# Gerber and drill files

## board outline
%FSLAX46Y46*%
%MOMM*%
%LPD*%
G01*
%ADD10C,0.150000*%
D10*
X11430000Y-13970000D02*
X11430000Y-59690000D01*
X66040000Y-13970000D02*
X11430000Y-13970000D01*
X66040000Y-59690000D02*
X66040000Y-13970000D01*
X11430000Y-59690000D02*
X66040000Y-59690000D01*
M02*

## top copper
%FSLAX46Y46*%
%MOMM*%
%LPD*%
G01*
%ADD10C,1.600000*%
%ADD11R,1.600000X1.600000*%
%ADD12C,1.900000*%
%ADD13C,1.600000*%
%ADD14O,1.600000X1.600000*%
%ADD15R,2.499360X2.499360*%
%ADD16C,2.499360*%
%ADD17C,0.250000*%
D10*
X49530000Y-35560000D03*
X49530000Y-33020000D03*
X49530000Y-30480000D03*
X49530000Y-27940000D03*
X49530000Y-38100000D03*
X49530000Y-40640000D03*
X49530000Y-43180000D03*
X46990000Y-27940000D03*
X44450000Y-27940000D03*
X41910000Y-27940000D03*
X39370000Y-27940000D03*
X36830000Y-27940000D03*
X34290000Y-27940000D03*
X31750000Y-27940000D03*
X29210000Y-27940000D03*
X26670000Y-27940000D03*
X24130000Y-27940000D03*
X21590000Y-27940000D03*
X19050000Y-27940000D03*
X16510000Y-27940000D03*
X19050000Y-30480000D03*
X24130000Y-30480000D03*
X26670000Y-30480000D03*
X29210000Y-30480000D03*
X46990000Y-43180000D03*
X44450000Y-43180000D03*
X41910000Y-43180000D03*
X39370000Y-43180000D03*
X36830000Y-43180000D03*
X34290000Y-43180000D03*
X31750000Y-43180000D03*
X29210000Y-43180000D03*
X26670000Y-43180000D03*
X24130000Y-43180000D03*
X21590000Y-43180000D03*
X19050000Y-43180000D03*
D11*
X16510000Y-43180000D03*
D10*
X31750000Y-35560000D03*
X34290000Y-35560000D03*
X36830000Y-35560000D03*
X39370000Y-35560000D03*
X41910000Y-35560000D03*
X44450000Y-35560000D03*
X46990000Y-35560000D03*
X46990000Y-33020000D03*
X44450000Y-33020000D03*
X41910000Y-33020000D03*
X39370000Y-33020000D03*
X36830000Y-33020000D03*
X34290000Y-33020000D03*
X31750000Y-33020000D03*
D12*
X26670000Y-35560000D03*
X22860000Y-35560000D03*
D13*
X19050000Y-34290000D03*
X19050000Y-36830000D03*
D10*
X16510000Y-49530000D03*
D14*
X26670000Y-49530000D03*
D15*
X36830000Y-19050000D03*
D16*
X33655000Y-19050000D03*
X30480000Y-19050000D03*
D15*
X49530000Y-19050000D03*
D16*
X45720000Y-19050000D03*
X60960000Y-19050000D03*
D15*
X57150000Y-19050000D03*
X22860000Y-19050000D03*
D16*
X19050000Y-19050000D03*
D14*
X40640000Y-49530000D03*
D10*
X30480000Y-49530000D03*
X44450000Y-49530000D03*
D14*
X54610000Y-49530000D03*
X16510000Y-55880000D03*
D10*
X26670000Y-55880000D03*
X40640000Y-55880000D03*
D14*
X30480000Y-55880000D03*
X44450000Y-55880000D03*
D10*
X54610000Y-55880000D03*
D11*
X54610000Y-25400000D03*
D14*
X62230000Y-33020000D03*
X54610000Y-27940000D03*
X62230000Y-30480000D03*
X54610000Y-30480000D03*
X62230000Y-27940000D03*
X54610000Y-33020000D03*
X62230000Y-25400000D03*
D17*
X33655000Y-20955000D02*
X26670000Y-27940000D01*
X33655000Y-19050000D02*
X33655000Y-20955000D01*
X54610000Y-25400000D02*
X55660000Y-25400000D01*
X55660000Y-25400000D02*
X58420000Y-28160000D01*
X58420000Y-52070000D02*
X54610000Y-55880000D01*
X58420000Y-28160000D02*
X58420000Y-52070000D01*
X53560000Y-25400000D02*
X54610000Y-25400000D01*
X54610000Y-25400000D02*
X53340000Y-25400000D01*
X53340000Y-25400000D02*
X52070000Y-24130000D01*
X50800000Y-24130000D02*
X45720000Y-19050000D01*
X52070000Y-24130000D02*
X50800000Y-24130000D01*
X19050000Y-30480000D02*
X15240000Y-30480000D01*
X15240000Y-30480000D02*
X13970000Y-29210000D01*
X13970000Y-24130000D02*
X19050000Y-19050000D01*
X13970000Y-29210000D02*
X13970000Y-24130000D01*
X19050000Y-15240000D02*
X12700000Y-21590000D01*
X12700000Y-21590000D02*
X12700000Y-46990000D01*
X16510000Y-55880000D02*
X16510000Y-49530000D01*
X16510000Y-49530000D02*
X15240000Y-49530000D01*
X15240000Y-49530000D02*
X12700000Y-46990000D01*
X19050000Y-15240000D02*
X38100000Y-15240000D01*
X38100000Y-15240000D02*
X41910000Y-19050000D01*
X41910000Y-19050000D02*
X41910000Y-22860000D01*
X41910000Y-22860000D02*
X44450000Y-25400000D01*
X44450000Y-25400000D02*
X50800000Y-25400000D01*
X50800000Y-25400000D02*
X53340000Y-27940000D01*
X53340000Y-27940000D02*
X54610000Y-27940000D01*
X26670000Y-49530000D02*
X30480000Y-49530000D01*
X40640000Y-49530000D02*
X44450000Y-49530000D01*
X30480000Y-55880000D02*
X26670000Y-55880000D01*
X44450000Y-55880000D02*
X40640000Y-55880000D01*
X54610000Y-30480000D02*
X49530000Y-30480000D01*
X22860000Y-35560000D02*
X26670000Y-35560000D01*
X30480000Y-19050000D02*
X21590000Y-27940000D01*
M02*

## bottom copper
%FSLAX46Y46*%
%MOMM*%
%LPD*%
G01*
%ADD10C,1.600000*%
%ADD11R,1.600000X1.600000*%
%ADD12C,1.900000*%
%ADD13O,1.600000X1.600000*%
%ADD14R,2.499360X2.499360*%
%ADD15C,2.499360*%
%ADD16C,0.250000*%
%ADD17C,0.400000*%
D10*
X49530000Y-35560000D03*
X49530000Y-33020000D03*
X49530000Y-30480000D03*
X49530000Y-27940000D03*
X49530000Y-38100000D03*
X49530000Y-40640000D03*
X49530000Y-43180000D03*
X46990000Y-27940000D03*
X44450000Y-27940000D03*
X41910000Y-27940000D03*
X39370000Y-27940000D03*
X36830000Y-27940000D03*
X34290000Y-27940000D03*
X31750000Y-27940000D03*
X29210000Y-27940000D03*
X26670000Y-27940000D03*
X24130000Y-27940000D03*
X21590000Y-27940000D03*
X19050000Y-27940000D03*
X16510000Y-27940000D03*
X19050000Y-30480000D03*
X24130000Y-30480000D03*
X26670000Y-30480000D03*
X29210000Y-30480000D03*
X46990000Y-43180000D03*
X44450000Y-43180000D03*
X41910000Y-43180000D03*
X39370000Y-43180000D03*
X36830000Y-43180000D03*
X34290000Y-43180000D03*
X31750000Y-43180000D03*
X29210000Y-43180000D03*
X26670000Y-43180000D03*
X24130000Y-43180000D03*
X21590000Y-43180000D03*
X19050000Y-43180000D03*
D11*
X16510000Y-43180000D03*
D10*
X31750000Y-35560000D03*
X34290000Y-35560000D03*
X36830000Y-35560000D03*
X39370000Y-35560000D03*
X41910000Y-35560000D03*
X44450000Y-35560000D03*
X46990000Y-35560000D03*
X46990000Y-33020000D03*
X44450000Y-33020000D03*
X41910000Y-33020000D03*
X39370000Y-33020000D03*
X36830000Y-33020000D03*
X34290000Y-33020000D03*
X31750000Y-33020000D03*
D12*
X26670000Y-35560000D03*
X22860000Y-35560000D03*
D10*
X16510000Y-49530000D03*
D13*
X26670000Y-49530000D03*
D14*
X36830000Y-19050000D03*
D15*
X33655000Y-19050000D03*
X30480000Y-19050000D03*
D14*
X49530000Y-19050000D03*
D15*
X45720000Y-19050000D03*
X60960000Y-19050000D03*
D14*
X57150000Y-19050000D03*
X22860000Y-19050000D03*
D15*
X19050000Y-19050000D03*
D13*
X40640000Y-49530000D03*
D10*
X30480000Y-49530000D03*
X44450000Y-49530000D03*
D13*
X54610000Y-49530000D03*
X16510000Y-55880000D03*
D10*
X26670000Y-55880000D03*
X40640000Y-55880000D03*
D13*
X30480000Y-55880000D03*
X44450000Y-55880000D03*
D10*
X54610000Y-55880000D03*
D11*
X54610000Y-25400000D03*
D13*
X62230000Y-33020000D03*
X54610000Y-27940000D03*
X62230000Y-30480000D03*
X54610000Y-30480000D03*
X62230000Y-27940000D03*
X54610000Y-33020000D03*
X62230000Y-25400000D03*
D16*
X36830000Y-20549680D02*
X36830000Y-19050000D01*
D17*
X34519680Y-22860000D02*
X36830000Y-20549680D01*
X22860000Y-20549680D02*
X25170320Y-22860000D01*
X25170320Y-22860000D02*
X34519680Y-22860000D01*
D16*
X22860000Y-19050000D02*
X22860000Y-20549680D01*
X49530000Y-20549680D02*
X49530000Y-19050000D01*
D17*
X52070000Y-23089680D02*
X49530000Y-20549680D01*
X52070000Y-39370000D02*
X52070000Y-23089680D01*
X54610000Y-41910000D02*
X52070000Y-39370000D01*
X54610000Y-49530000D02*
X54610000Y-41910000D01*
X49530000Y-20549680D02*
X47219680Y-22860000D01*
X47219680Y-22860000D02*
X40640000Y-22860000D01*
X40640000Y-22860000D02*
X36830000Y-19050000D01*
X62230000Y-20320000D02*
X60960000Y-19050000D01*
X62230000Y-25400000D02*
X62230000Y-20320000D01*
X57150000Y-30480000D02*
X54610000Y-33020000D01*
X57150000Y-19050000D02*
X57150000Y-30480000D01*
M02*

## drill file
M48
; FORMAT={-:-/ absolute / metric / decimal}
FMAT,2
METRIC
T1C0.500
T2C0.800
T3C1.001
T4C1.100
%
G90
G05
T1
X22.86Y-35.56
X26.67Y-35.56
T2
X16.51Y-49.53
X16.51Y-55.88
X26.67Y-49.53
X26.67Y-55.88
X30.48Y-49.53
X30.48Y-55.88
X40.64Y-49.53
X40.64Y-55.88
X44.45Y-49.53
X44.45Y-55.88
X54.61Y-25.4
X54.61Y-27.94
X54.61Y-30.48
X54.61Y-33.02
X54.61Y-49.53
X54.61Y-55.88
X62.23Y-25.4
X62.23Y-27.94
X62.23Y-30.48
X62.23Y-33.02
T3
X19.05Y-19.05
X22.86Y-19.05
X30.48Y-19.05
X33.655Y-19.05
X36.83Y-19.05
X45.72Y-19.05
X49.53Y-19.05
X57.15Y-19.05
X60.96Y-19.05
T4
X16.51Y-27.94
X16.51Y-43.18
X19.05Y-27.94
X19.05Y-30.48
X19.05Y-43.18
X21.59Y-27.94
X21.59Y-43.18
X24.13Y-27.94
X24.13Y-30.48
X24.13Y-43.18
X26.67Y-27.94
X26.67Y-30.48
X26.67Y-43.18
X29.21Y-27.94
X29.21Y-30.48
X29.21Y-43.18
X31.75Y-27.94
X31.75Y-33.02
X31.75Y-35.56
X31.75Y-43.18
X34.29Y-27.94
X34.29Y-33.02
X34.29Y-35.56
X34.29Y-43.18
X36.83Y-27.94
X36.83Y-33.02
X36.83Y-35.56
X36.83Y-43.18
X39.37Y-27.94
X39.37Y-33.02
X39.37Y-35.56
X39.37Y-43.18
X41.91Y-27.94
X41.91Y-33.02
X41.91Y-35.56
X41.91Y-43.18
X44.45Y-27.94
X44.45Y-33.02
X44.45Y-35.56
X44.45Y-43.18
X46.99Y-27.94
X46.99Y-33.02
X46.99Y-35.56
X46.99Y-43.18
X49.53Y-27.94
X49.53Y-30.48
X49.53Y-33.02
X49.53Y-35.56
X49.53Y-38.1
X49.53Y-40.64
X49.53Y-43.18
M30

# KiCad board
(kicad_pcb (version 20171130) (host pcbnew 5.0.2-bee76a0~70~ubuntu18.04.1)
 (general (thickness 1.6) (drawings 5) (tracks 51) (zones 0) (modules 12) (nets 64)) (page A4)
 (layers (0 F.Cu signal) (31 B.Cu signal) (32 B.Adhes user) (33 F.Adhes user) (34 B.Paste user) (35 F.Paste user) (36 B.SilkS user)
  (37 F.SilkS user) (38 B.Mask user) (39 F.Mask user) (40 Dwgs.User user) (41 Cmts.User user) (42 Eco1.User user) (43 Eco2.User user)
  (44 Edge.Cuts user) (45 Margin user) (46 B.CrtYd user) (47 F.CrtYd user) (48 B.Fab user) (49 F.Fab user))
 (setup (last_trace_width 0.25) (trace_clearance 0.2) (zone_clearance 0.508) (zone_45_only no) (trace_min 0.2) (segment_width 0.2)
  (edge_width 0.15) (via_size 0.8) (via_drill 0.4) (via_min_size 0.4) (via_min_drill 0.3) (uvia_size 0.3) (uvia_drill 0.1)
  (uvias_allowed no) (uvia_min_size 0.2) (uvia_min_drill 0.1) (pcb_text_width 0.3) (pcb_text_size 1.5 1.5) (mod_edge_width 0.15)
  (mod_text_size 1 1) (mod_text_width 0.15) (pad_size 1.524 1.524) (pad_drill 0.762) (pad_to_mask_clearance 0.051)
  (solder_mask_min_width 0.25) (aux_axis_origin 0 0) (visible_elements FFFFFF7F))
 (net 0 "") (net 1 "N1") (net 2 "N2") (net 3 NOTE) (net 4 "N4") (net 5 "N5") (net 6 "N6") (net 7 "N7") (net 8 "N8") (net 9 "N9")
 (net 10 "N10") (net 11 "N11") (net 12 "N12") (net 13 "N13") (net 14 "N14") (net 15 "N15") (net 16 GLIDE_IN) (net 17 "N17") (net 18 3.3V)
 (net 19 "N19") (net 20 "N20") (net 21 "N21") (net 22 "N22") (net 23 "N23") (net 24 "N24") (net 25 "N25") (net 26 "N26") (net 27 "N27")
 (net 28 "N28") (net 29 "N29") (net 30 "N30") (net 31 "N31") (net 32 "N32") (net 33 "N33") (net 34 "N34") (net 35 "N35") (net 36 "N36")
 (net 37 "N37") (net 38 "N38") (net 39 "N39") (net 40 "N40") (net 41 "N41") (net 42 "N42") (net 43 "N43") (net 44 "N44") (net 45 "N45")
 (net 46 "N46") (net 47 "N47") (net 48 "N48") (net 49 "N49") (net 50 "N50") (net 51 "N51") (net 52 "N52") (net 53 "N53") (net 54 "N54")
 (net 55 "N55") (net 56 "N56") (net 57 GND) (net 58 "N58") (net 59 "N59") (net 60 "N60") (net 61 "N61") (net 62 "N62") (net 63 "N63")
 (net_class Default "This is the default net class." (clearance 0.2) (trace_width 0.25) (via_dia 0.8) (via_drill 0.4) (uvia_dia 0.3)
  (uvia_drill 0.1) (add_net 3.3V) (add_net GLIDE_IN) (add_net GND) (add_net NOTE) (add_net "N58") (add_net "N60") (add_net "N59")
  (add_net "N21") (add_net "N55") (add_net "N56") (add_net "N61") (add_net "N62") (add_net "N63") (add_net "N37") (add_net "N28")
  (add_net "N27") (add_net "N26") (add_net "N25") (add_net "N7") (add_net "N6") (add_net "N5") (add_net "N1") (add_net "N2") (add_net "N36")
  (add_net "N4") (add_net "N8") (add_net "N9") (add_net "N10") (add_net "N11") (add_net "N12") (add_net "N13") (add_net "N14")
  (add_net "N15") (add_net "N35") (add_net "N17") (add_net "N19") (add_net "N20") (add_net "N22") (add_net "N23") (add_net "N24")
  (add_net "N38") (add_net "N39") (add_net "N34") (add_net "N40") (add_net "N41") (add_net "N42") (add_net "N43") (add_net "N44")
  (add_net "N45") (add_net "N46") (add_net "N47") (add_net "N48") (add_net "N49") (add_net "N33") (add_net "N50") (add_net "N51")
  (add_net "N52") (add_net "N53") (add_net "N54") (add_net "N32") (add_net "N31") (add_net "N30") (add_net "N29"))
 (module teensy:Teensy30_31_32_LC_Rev (layer F.Cu) (at 33.02 35.56)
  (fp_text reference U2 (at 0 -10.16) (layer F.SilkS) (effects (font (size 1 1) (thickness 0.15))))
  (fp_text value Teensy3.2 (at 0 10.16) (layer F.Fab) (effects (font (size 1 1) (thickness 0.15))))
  (pad 17 thru_hole circle (at 16.51 0) (size 1.6 1.6) (drill 1.1) (layers *.Cu *.Mask F.SilkS) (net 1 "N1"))
  (pad 18 thru_hole circle (at 16.51 -2.54) (size 1.6 1.6) (drill 1.1) (layers *.Cu *.Mask F.SilkS) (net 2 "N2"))
  (pad 19 thru_hole circle (at 16.51 -5.08) (size 1.6 1.6) (drill 1.1) (layers *.Cu *.Mask F.SilkS) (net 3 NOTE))
  (pad 20 thru_hole circle (at 16.51 -7.62) (size 1.6 1.6) (drill 1.1) (layers *.Cu *.Mask F.SilkS) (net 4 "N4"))
  (pad 16 thru_hole circle (at 16.51 2.54) (size 1.6 1.6) (drill 1.1) (layers *.Cu *.Mask F.SilkS) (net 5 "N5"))
  (pad 15 thru_hole circle (at 16.51 5.08) (size 1.6 1.6) (drill 1.1) (layers *.Cu *.Mask F.SilkS) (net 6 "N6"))
  (pad 14 thru_hole circle (at 16.51 7.62) (size 1.6 1.6) (drill 1.1) (layers *.Cu *.Mask F.SilkS) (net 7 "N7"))
  (pad 21 thru_hole circle (at 13.97 -7.62) (size 1.6 1.6) (drill 1.1) (layers *.Cu *.Mask F.SilkS) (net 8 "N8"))
  (pad 22 thru_hole circle (at 11.43 -7.62) (size 1.6 1.6) (drill 1.1) (layers *.Cu *.Mask F.SilkS) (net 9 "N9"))
  (pad 23 thru_hole circle (at 8.89 -7.62) (size 1.6 1.6) (drill 1.1) (layers *.Cu *.Mask F.SilkS) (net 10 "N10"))
  (pad 24 thru_hole circle (at 6.35 -7.62) (size 1.6 1.6) (drill 1.1) (layers *.Cu *.Mask F.SilkS) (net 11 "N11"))
  (pad 25 thru_hole circle (at 3.81 -7.62) (size 1.6 1.6) (drill 1.1) (layers *.Cu *.Mask F.SilkS) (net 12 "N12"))
  (pad 26 thru_hole circle (at 1.27 -7.62) (size 1.6 1.6) (drill 1.1) (layers *.Cu *.Mask F.SilkS) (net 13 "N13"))
  (pad 27 thru_hole circle (at -1.27 -7.62) (size 1.6 1.6) (drill 1.1) (layers *.Cu *.Mask F.SilkS) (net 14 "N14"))
  (pad 28 thru_hole circle (at -3.81 -7.62) (size 1.6 1.6) (drill 1.1) (layers *.Cu *.Mask F.SilkS) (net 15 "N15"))
  (pad 29 thru_hole circle (at -6.35 -7.62) (size 1.6 1.6) (drill 1.1) (layers *.Cu *.Mask F.SilkS) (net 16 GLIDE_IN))
  (pad 30 thru_hole circle (at -8.89 -7.62) (size 1.6 1.6) (drill 1.1) (layers *.Cu *.Mask F.SilkS) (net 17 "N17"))
  (pad 31 thru_hole circle (at -11.43 -7.62) (size 1.6 1.6) (drill 1.1) (layers *.Cu *.Mask F.SilkS) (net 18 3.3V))
  (pad 32 thru_hole circle (at -13.97 -7.62) (size 1.6 1.6) (drill 1.1) (layers *.Cu *.Mask F.SilkS) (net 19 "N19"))
  (pad 33 thru_hole circle (at -16.51 -7.62) (size 1.6 1.6) (drill 1.1) (layers *.Cu *.Mask F.SilkS) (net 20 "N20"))
  (pad 34 thru_hole circle (at -13.97 -5.08) (size 1.6 1.6) (drill 1.1) (layers *.Cu *.Mask F.SilkS) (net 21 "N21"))
  (pad 35 thru_hole circle (at -8.89 -5.08) (size 1.6 1.6) (drill 1.1) (layers *.Cu *.Mask F.SilkS) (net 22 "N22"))
  (pad 36 thru_hole circle (at -6.35 -5.08) (size 1.6 1.6) (drill 1.1) (layers *.Cu *.Mask F.SilkS) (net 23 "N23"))
  (pad 37 thru_hole circle (at -3.81 -5.08) (size 1.6 1.6) (drill 1.1) (layers *.Cu *.Mask F.SilkS) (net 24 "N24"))
  (pad 13 thru_hole circle (at 13.97 7.62) (size 1.6 1.6) (drill 1.1) (layers *.Cu *.Mask F.SilkS) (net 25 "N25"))
  (pad 12 thru_hole circle (at 11.43 7.62) (size 1.6 1.6) (drill 1.1) (layers *.Cu *.Mask F.SilkS) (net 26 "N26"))
  (pad 11 thru_hole circle (at 8.89 7.62) (size 1.6 1.6) (drill 1.1) (layers *.Cu *.Mask F.SilkS) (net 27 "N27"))
  (pad 10 thru_hole circle (at 6.35 7.62) (size 1.6 1.6) (drill 1.1) (layers *.Cu *.Mask F.SilkS) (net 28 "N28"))
  (pad 9 thru_hole circle (at 3.81 7.62) (size 1.6 1.6) (drill 1.1) (layers *.Cu *.Mask F.SilkS) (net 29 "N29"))
  (pad 8 thru_hole circle (at 1.27 7.62) (size 1.6 1.6) (drill 1.1) (layers *.Cu *.Mask F.SilkS) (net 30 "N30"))
  (pad 7 thru_hole circle (at -1.27 7.62) (size 1.6 1.6) (drill 1.1) (layers *.Cu *.Mask F.SilkS) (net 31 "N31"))
  (pad 6 thru_hole circle (at -3.81 7.62) (size 1.6 1.6) (drill 1.1) (layers *.Cu *.Mask F.SilkS) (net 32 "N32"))
  (pad 5 thru_hole circle (at -6.35 7.62) (size 1.6 1.6) (drill 1.1) (layers *.Cu *.Mask F.SilkS) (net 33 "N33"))
  (pad 4 thru_hole circle (at -8.89 7.62) (size 1.6 1.6) (drill 1.1) (layers *.Cu *.Mask F.SilkS) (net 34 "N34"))
  (pad 3 thru_hole circle (at -11.43 7.62) (size 1.6 1.6) (drill 1.1) (layers *.Cu *.Mask F.SilkS) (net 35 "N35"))
  (pad 2 thru_hole circle (at -13.97 7.62) (size 1.6 1.6) (drill 1.1) (layers *.Cu *.Mask F.SilkS) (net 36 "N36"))
  (pad 1 thru_hole rect (at -16.51 7.62) (size 1.6 1.6) (drill 1.1) (layers *.Cu *.Mask F.SilkS) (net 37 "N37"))
  (pad 38 thru_hole circle (at -1.27 0) (size 1.6 1.6) (drill 1.1) (layers *.Cu *.Mask) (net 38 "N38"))
  (pad 39 thru_hole circle (at 1.27 0) (size 1.6 1.6) (drill 1.1) (layers *.Cu *.Mask) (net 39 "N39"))
  (pad 40 thru_hole circle (at 3.81 0) (size 1.6 1.6) (drill 1.1) (layers *.Cu *.Mask) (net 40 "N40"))
  (pad 41 thru_hole circle (at 6.35 0) (size 1.6 1.6) (drill 1.1) (layers *.Cu *.Mask) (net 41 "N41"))
  (pad 42 thru_hole circle (at 8.89 0) (size 1.6 1.6) (drill 1.1) (layers *.Cu *.Mask) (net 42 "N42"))
  (pad 43 thru_hole circle (at 11.43 0) (size 1.6 1.6) (drill 1.1) (layers *.Cu *.Mask) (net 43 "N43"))
  (pad 44 thru_hole circle (at 13.97 0) (size 1.6 1.6) (drill 1.1) (layers *.Cu *.Mask) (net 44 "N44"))
  (pad 45 thru_hole circle (at 13.97 -2.54) (size 1.6 1.6) (drill 1.1) (layers *.Cu *.Mask) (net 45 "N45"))
  (pad 46 thru_hole circle (at 11.43 -2.54) (size 1.6 1.6) (drill 1.1) (layers *.Cu *.Mask) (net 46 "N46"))
  (pad 47 thru_hole circle (at 8.89 -2.54) (size 1.6 1.6) (drill 1.1) (layers *.Cu *.Mask) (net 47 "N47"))
  (pad 48 thru_hole circle (at 6.35 -2.54) (size 1.6 1.6) (drill 1.1) (layers *.Cu *.Mask) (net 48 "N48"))
  (pad 49 thru_hole circle (at 3.81 -2.54) (size 1.6 1.6) (drill 1.1) (layers *.Cu *.Mask) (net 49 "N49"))
  (pad 50 thru_hole circle (at 1.27 -2.54) (size 1.6 1.6) (drill 1.1) (layers *.Cu *.Mask) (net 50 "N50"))
  (pad 51 thru_hole circle (at -1.27 -2.54) (size 1.6 1.6) (drill 1.1) (layers *.Cu *.Mask) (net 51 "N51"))
  (pad 52 thru_hole circle (at -6.35 0) (size 1.9 1.9) (drill 0.5) (layers *.Cu *.Mask F.SilkS) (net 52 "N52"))
  (pad 52 thru_hole circle (at -10.16 0) (size 1.9 1.9) (drill 0.5) (layers *.Cu *.Mask F.SilkS) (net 52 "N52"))
  (pad 53 smd circle (at -13.97 -1.27) (size 1.6 1.6) (layers F.Cu F.Paste F.Mask) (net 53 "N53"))
  (pad 54 smd circle (at -13.97 1.27) (size 1.6 1.6) (layers F.Cu F.Paste F.Mask) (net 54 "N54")))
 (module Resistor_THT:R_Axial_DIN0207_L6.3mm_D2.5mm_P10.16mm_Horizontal (layer F.Cu) (at 16.51 49.53)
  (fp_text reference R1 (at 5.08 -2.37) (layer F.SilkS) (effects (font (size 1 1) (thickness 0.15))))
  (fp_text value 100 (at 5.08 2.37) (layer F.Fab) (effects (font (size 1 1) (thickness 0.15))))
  (pad 1 thru_hole circle (at 0 0) (size 1.6 1.6) (drill 0.8) (layers *.Cu *.Mask) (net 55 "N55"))
  (pad 2 thru_hole oval (at 10.16 0) (size 1.6 1.6) (drill 0.8) (layers *.Cu *.Mask) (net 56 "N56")))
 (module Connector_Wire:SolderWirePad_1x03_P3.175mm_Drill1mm (layer F.Cu) (at 36.83 19.05 180)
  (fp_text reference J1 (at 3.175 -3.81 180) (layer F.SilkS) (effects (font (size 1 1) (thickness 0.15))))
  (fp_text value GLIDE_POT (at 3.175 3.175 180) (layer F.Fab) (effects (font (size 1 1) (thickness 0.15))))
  (pad 1 thru_hole rect (at 0 0 180) (size 2.49936 2.49936) (drill 1.00076) (layers *.Cu *.Mask) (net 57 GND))
  (pad 2 thru_hole circle (at 3.175 0 180) (size 2.49936 2.49936) (drill 1.00076) (layers *.Cu *.Mask) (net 16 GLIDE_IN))
  (pad 3 thru_hole circle (at 6.35 0 180) (size 2.49936 2.49936) (drill 1.00076) (layers *.Cu *.Mask) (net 18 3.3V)))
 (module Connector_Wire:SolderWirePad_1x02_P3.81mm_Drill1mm (layer F.Cu) (at 49.53 19.05 180)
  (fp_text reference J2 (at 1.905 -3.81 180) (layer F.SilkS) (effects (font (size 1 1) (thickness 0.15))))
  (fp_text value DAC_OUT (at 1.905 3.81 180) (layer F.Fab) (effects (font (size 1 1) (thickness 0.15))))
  (pad 1 thru_hole rect (at 0 0 180) (size 2.49936 2.49936) (drill 1.00076) (layers *.Cu *.Mask) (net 57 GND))
  (pad 2 thru_hole circle (at 3.81 0 180) (size 2.49936 2.49936) (drill 1.00076) (layers *.Cu *.Mask) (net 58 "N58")))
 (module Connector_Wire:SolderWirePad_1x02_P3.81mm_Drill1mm (layer F.Cu) (at 57.15 19.05)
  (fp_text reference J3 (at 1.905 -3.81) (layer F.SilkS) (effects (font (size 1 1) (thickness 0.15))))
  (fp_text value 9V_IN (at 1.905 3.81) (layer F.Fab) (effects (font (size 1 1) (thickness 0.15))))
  (pad 2 thru_hole circle (at 3.81 0) (size 2.49936 2.49936) (drill 1.00076) (layers *.Cu *.Mask) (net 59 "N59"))
  (pad 1 thru_hole rect (at 0 0) (size 2.49936 2.49936) (drill 1.00076) (layers *.Cu *.Mask) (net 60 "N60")))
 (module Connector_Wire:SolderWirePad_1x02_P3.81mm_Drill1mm (layer F.Cu) (at 22.86 19.05 180)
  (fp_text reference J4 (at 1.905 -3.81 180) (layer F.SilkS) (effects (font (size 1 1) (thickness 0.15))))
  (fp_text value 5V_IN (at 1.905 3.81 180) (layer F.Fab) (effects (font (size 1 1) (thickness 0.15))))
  (pad 1 thru_hole rect (at 0 0 180) (size 2.49936 2.49936) (drill 1.00076) (layers *.Cu *.Mask) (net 57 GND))
  (pad 2 thru_hole circle (at 3.81 0 180) (size 2.49936 2.49936) (drill 1.00076) (layers *.Cu *.Mask) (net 21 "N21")))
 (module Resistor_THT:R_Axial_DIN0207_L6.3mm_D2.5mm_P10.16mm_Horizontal (layer F.Cu) (at 30.48 49.53)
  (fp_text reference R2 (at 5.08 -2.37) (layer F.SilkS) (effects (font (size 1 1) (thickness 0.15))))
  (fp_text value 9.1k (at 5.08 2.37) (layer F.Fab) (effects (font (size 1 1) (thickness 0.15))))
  (pad 2 thru_hole oval (at 10.16 0) (size 1.6 1.6) (drill 0.8) (layers *.Cu *.Mask) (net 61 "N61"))
  (pad 1 thru_hole circle (at 0 0) (size 1.6 1.6) (drill 0.8) (layers *.Cu *.Mask) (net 56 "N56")))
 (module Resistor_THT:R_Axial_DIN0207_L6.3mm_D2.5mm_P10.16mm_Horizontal (layer F.Cu) (at 44.45 49.53)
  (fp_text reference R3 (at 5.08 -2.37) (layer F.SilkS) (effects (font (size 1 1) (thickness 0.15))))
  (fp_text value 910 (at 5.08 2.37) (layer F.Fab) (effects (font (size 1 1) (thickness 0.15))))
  (pad 1 thru_hole circle (at 0 0) (size 1.6 1.6) (drill 0.8) (layers *.Cu *.Mask) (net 61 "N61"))
  (pad 2 thru_hole oval (at 10.16 0) (size 1.6 1.6) (drill 0.8) (layers *.Cu *.Mask) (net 57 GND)))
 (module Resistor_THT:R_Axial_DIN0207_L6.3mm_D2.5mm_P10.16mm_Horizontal (layer F.Cu) (at 26.67 55.88 180)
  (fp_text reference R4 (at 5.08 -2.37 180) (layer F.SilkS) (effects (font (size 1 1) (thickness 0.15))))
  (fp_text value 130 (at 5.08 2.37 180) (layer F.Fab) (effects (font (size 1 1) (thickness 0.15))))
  (pad 2 thru_hole oval (at 10.16 0 180) (size 1.6 1.6) (drill 0.8) (layers *.Cu *.Mask) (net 55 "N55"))
  (pad 1 thru_hole circle (at 0 0 180) (size 1.6 1.6) (drill 0.8) (layers *.Cu *.Mask) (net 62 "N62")))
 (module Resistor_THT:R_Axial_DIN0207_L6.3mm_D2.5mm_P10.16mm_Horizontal (layer F.Cu) (at 40.64 55.88 180)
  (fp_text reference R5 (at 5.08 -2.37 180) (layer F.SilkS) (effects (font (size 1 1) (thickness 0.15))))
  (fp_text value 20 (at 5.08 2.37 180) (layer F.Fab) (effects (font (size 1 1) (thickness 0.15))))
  (pad 1 thru_hole circle (at 0 0 180) (size 1.6 1.6) (drill 0.8) (layers *.Cu *.Mask) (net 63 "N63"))
  (pad 2 thru_hole oval (at 10.16 0 180) (size 1.6 1.6) (drill 0.8) (layers *.Cu *.Mask) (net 62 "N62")))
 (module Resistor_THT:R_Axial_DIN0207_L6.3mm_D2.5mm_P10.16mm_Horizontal (layer F.Cu) (at 54.61 55.88 180)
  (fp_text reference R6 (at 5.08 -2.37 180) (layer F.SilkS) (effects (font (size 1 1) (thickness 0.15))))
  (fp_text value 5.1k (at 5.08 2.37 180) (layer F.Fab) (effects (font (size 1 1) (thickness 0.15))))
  (pad 2 thru_hole oval (at 10.16 0 180) (size 1.6 1.6) (drill 0.8) (layers *.Cu *.Mask) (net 63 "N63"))
  (pad 1 thru_hole circle (at 0 0 180) (size 1.6 1.6) (drill 0.8) (layers *.Cu *.Mask) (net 58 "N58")))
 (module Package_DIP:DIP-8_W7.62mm (layer F.Cu) (at 54.61 25.4)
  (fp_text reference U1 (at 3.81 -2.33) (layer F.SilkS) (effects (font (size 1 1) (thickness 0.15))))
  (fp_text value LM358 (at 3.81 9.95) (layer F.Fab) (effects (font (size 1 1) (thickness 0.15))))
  (pad 1 thru_hole rect (at 0 0) (size 1.6 1.6) (drill 0.8) (layers *.Cu *.Mask) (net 58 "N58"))
  (pad 5 thru_hole oval (at 7.62 7.62) (size 1.6 1.6) (drill 0.8) (layers *.Cu *.Mask))
  (pad 2 thru_hole oval (at 0 2.54) (size 1.6 1.6) (drill 0.8) (layers *.Cu *.Mask) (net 55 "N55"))
  (pad 6 thru_hole oval (at 7.62 5.08) (size 1.6 1.6) (drill 0.8) (layers *.Cu *.Mask))
  (pad 3 thru_hole oval (at 0 5.08) (size 1.6 1.6) (drill 0.8) (layers *.Cu *.Mask) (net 3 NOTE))
  (pad 7 thru_hole oval (at 7.62 2.54) (size 1.6 1.6) (drill 0.8) (layers *.Cu *.Mask))
  (pad 4 thru_hole oval (at 0 7.62) (size 1.6 1.6) (drill 0.8) (layers *.Cu *.Mask) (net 60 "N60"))
  (pad 8 thru_hole oval (at 7.62 0) (size 1.6 1.6) (drill 0.8) (layers *.Cu *.Mask) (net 59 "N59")))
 (gr_line (start 11.43 13.97) (end 11.43 59.69) (layer Edge.Cuts) (width 0.15))
 (gr_line (start 66.04 13.97) (end 11.43 13.97) (layer Edge.Cuts) (width 0.15))
 (gr_line (start 66.04 59.69) (end 66.04 13.97) (layer Edge.Cuts) (width 0.15))
 (gr_line (start 11.43 59.69) (end 66.04 59.69) (layer Edge.Cuts) (width 0.15))
 (segment (start 36.83 20.54968) (end 36.83 19.05) (width 0.25) (layer B.Cu) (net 57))
 (segment (start 34.51968 22.86) (end 36.83 20.54968) (width 0.4) (layer B.Cu) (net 57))
 (segment (start 22.86 20.54968) (end 25.17032 22.86) (width 0.4) (layer B.Cu) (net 57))
 (segment (start 25.17032 22.86) (end 34.51968 22.86) (width 0.4) (layer B.Cu) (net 57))
 (segment (start 22.86 19.05) (end 22.86 20.54968) (width 0.25) (layer B.Cu) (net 57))
 (segment (start 49.53 20.54968) (end 49.53 19.05) (width 0.25) (layer B.Cu) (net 57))
 (segment (start 52.07 23.08968) (end 49.53 20.54968) (width 0.4) (layer B.Cu) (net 57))
 (segment (start 52.07 39.37) (end 52.07 23.08968) (width 0.4) (layer B.Cu) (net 57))
 (segment (start 54.61 41.91) (end 52.07 39.37) (width 0.4) (layer B.Cu) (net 57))
 (segment (start 54.61 49.53) (end 54.61 41.91) (width 0.4) (layer B.Cu) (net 57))
 (segment (start 49.53 20.54968) (end 47.21968 22.86) (width 0.4) (layer B.Cu) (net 57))
 (segment (start 47.21968 22.86) (end 40.64 22.86) (width 0.4) (layer B.Cu) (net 57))
 (segment (start 40.64 22.86) (end 36.83 19.05) (width 0.4) (layer B.Cu) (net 57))
 (segment (start 33.655 20.955) (end 26.67 27.94) (width 0.25) (layer F.Cu) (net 16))
 (segment (start 33.655 19.05) (end 33.655 20.955) (width 0.25) (layer F.Cu) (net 16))
 (segment (start 54.61 25.4) (end 55.66 25.4) (width 0.25) (layer F.Cu) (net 58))
 (segment (start 55.66 25.4) (end 58.42 28.16) (width 0.25) (layer F.Cu) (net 58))
 (segment (start 58.42 52.07) (end 54.61 55.88) (width 0.25) (layer F.Cu) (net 58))
 (segment (start 58.42 28.16) (end 58.42 52.07) (width 0.25) (layer F.Cu) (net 58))
 (segment (start 53.56 25.4) (end 54.61 25.4) (width 0.25) (layer F.Cu) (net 58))
 (segment (start 54.61 25.4) (end 53.34 25.4) (width 0.25) (layer F.Cu) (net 58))
 (segment (start 53.34 25.4) (end 52.07 24.13) (width 0.25) (layer F.Cu) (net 58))
 (segment (start 50.8 24.13) (end 45.72 19.05) (width 0.25) (layer F.Cu) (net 58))
 (segment (start 52.07 24.13) (end 50.8 24.13) (width 0.25) (layer F.Cu) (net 58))
 (segment (start 62.23 20.32) (end 60.96 19.05) (width 0.4) (layer B.Cu) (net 59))
 (segment (start 62.23 25.4) (end 62.23 20.32) (width 0.4) (layer B.Cu) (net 59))
 (segment (start 57.15 30.48) (end 54.61 33.02) (width 0.4) (layer B.Cu) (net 60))
 (segment (start 57.15 19.05) (end 57.15 30.48) (width 0.4) (layer B.Cu) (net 60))
 (segment (start 19.05 30.48) (end 15.24 30.48) (width 0.25) (layer F.Cu) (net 21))
 (segment (start 15.24 30.48) (end 13.97 29.21) (width 0.25) (layer F.Cu) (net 21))
 (segment (start 13.97 24.13) (end 19.05 19.05) (width 0.25) (layer F.Cu) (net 21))
 (segment (start 13.97 29.21) (end 13.97 24.13) (width 0.25) (layer F.Cu) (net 21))
 (segment (start 19.05 15.24) (end 12.7 21.59) (width 0.25) (layer F.Cu) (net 55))
 (segment (start 12.7 21.59) (end 12.7 46.99) (width 0.25) (layer F.Cu) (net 55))
 (segment (start 16.51 55.88) (end 16.51 49.53) (width 0.25) (layer F.Cu) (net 55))
 (segment (start 16.51 49.53) (end 15.24 49.53) (width 0.25) (layer F.Cu) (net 55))
 (segment (start 15.24 49.53) (end 12.7 46.99) (width 0.25) (layer F.Cu) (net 55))
 (segment (start 19.05 15.24) (end 38.1 15.24) (width 0.25) (layer F.Cu) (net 55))
 (segment (start 38.1 15.24) (end 41.91 19.05) (width 0.25) (layer F.Cu) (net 55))
 (segment (start 41.91 19.05) (end 41.91 22.86) (width 0.25) (layer F.Cu) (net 55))
 (segment (start 41.91 22.86) (end 44.45 25.4) (width 0.25) (layer F.Cu) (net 55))
 (segment (start 44.45 25.4) (end 50.8 25.4) (width 0.25) (layer F.Cu) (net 55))
 (segment (start 50.8 25.4) (end 53.34 27.94) (width 0.25) (layer F.Cu) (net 55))
 (segment (start 53.34 27.94) (end 54.61 27.94) (width 0.25) (layer F.Cu) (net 55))
 (segment (start 26.67 49.53) (end 30.48 49.53) (width 0.25) (layer F.Cu) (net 56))
 (segment (start 40.64 49.53) (end 44.45 49.53) (width 0.25) (layer F.Cu) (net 61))
 (segment (start 30.48 55.88) (end 26.67 55.88) (width 0.25) (layer F.Cu) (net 62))
 (segment (start 44.45 55.88) (end 40.64 55.88) (width 0.25) (layer F.Cu) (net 63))
 (segment (start 54.61 30.48) (end 49.53 30.48) (width 0.25) (layer F.Cu) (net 3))
 (segment (start 22.86 35.56) (end 26.67 35.56) (width 0.25) (layer F.Cu) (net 52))
 (segment (start 30.48 19.05) (end 21.59 27.94) (width 0.25) (layer F.Cu) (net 18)))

